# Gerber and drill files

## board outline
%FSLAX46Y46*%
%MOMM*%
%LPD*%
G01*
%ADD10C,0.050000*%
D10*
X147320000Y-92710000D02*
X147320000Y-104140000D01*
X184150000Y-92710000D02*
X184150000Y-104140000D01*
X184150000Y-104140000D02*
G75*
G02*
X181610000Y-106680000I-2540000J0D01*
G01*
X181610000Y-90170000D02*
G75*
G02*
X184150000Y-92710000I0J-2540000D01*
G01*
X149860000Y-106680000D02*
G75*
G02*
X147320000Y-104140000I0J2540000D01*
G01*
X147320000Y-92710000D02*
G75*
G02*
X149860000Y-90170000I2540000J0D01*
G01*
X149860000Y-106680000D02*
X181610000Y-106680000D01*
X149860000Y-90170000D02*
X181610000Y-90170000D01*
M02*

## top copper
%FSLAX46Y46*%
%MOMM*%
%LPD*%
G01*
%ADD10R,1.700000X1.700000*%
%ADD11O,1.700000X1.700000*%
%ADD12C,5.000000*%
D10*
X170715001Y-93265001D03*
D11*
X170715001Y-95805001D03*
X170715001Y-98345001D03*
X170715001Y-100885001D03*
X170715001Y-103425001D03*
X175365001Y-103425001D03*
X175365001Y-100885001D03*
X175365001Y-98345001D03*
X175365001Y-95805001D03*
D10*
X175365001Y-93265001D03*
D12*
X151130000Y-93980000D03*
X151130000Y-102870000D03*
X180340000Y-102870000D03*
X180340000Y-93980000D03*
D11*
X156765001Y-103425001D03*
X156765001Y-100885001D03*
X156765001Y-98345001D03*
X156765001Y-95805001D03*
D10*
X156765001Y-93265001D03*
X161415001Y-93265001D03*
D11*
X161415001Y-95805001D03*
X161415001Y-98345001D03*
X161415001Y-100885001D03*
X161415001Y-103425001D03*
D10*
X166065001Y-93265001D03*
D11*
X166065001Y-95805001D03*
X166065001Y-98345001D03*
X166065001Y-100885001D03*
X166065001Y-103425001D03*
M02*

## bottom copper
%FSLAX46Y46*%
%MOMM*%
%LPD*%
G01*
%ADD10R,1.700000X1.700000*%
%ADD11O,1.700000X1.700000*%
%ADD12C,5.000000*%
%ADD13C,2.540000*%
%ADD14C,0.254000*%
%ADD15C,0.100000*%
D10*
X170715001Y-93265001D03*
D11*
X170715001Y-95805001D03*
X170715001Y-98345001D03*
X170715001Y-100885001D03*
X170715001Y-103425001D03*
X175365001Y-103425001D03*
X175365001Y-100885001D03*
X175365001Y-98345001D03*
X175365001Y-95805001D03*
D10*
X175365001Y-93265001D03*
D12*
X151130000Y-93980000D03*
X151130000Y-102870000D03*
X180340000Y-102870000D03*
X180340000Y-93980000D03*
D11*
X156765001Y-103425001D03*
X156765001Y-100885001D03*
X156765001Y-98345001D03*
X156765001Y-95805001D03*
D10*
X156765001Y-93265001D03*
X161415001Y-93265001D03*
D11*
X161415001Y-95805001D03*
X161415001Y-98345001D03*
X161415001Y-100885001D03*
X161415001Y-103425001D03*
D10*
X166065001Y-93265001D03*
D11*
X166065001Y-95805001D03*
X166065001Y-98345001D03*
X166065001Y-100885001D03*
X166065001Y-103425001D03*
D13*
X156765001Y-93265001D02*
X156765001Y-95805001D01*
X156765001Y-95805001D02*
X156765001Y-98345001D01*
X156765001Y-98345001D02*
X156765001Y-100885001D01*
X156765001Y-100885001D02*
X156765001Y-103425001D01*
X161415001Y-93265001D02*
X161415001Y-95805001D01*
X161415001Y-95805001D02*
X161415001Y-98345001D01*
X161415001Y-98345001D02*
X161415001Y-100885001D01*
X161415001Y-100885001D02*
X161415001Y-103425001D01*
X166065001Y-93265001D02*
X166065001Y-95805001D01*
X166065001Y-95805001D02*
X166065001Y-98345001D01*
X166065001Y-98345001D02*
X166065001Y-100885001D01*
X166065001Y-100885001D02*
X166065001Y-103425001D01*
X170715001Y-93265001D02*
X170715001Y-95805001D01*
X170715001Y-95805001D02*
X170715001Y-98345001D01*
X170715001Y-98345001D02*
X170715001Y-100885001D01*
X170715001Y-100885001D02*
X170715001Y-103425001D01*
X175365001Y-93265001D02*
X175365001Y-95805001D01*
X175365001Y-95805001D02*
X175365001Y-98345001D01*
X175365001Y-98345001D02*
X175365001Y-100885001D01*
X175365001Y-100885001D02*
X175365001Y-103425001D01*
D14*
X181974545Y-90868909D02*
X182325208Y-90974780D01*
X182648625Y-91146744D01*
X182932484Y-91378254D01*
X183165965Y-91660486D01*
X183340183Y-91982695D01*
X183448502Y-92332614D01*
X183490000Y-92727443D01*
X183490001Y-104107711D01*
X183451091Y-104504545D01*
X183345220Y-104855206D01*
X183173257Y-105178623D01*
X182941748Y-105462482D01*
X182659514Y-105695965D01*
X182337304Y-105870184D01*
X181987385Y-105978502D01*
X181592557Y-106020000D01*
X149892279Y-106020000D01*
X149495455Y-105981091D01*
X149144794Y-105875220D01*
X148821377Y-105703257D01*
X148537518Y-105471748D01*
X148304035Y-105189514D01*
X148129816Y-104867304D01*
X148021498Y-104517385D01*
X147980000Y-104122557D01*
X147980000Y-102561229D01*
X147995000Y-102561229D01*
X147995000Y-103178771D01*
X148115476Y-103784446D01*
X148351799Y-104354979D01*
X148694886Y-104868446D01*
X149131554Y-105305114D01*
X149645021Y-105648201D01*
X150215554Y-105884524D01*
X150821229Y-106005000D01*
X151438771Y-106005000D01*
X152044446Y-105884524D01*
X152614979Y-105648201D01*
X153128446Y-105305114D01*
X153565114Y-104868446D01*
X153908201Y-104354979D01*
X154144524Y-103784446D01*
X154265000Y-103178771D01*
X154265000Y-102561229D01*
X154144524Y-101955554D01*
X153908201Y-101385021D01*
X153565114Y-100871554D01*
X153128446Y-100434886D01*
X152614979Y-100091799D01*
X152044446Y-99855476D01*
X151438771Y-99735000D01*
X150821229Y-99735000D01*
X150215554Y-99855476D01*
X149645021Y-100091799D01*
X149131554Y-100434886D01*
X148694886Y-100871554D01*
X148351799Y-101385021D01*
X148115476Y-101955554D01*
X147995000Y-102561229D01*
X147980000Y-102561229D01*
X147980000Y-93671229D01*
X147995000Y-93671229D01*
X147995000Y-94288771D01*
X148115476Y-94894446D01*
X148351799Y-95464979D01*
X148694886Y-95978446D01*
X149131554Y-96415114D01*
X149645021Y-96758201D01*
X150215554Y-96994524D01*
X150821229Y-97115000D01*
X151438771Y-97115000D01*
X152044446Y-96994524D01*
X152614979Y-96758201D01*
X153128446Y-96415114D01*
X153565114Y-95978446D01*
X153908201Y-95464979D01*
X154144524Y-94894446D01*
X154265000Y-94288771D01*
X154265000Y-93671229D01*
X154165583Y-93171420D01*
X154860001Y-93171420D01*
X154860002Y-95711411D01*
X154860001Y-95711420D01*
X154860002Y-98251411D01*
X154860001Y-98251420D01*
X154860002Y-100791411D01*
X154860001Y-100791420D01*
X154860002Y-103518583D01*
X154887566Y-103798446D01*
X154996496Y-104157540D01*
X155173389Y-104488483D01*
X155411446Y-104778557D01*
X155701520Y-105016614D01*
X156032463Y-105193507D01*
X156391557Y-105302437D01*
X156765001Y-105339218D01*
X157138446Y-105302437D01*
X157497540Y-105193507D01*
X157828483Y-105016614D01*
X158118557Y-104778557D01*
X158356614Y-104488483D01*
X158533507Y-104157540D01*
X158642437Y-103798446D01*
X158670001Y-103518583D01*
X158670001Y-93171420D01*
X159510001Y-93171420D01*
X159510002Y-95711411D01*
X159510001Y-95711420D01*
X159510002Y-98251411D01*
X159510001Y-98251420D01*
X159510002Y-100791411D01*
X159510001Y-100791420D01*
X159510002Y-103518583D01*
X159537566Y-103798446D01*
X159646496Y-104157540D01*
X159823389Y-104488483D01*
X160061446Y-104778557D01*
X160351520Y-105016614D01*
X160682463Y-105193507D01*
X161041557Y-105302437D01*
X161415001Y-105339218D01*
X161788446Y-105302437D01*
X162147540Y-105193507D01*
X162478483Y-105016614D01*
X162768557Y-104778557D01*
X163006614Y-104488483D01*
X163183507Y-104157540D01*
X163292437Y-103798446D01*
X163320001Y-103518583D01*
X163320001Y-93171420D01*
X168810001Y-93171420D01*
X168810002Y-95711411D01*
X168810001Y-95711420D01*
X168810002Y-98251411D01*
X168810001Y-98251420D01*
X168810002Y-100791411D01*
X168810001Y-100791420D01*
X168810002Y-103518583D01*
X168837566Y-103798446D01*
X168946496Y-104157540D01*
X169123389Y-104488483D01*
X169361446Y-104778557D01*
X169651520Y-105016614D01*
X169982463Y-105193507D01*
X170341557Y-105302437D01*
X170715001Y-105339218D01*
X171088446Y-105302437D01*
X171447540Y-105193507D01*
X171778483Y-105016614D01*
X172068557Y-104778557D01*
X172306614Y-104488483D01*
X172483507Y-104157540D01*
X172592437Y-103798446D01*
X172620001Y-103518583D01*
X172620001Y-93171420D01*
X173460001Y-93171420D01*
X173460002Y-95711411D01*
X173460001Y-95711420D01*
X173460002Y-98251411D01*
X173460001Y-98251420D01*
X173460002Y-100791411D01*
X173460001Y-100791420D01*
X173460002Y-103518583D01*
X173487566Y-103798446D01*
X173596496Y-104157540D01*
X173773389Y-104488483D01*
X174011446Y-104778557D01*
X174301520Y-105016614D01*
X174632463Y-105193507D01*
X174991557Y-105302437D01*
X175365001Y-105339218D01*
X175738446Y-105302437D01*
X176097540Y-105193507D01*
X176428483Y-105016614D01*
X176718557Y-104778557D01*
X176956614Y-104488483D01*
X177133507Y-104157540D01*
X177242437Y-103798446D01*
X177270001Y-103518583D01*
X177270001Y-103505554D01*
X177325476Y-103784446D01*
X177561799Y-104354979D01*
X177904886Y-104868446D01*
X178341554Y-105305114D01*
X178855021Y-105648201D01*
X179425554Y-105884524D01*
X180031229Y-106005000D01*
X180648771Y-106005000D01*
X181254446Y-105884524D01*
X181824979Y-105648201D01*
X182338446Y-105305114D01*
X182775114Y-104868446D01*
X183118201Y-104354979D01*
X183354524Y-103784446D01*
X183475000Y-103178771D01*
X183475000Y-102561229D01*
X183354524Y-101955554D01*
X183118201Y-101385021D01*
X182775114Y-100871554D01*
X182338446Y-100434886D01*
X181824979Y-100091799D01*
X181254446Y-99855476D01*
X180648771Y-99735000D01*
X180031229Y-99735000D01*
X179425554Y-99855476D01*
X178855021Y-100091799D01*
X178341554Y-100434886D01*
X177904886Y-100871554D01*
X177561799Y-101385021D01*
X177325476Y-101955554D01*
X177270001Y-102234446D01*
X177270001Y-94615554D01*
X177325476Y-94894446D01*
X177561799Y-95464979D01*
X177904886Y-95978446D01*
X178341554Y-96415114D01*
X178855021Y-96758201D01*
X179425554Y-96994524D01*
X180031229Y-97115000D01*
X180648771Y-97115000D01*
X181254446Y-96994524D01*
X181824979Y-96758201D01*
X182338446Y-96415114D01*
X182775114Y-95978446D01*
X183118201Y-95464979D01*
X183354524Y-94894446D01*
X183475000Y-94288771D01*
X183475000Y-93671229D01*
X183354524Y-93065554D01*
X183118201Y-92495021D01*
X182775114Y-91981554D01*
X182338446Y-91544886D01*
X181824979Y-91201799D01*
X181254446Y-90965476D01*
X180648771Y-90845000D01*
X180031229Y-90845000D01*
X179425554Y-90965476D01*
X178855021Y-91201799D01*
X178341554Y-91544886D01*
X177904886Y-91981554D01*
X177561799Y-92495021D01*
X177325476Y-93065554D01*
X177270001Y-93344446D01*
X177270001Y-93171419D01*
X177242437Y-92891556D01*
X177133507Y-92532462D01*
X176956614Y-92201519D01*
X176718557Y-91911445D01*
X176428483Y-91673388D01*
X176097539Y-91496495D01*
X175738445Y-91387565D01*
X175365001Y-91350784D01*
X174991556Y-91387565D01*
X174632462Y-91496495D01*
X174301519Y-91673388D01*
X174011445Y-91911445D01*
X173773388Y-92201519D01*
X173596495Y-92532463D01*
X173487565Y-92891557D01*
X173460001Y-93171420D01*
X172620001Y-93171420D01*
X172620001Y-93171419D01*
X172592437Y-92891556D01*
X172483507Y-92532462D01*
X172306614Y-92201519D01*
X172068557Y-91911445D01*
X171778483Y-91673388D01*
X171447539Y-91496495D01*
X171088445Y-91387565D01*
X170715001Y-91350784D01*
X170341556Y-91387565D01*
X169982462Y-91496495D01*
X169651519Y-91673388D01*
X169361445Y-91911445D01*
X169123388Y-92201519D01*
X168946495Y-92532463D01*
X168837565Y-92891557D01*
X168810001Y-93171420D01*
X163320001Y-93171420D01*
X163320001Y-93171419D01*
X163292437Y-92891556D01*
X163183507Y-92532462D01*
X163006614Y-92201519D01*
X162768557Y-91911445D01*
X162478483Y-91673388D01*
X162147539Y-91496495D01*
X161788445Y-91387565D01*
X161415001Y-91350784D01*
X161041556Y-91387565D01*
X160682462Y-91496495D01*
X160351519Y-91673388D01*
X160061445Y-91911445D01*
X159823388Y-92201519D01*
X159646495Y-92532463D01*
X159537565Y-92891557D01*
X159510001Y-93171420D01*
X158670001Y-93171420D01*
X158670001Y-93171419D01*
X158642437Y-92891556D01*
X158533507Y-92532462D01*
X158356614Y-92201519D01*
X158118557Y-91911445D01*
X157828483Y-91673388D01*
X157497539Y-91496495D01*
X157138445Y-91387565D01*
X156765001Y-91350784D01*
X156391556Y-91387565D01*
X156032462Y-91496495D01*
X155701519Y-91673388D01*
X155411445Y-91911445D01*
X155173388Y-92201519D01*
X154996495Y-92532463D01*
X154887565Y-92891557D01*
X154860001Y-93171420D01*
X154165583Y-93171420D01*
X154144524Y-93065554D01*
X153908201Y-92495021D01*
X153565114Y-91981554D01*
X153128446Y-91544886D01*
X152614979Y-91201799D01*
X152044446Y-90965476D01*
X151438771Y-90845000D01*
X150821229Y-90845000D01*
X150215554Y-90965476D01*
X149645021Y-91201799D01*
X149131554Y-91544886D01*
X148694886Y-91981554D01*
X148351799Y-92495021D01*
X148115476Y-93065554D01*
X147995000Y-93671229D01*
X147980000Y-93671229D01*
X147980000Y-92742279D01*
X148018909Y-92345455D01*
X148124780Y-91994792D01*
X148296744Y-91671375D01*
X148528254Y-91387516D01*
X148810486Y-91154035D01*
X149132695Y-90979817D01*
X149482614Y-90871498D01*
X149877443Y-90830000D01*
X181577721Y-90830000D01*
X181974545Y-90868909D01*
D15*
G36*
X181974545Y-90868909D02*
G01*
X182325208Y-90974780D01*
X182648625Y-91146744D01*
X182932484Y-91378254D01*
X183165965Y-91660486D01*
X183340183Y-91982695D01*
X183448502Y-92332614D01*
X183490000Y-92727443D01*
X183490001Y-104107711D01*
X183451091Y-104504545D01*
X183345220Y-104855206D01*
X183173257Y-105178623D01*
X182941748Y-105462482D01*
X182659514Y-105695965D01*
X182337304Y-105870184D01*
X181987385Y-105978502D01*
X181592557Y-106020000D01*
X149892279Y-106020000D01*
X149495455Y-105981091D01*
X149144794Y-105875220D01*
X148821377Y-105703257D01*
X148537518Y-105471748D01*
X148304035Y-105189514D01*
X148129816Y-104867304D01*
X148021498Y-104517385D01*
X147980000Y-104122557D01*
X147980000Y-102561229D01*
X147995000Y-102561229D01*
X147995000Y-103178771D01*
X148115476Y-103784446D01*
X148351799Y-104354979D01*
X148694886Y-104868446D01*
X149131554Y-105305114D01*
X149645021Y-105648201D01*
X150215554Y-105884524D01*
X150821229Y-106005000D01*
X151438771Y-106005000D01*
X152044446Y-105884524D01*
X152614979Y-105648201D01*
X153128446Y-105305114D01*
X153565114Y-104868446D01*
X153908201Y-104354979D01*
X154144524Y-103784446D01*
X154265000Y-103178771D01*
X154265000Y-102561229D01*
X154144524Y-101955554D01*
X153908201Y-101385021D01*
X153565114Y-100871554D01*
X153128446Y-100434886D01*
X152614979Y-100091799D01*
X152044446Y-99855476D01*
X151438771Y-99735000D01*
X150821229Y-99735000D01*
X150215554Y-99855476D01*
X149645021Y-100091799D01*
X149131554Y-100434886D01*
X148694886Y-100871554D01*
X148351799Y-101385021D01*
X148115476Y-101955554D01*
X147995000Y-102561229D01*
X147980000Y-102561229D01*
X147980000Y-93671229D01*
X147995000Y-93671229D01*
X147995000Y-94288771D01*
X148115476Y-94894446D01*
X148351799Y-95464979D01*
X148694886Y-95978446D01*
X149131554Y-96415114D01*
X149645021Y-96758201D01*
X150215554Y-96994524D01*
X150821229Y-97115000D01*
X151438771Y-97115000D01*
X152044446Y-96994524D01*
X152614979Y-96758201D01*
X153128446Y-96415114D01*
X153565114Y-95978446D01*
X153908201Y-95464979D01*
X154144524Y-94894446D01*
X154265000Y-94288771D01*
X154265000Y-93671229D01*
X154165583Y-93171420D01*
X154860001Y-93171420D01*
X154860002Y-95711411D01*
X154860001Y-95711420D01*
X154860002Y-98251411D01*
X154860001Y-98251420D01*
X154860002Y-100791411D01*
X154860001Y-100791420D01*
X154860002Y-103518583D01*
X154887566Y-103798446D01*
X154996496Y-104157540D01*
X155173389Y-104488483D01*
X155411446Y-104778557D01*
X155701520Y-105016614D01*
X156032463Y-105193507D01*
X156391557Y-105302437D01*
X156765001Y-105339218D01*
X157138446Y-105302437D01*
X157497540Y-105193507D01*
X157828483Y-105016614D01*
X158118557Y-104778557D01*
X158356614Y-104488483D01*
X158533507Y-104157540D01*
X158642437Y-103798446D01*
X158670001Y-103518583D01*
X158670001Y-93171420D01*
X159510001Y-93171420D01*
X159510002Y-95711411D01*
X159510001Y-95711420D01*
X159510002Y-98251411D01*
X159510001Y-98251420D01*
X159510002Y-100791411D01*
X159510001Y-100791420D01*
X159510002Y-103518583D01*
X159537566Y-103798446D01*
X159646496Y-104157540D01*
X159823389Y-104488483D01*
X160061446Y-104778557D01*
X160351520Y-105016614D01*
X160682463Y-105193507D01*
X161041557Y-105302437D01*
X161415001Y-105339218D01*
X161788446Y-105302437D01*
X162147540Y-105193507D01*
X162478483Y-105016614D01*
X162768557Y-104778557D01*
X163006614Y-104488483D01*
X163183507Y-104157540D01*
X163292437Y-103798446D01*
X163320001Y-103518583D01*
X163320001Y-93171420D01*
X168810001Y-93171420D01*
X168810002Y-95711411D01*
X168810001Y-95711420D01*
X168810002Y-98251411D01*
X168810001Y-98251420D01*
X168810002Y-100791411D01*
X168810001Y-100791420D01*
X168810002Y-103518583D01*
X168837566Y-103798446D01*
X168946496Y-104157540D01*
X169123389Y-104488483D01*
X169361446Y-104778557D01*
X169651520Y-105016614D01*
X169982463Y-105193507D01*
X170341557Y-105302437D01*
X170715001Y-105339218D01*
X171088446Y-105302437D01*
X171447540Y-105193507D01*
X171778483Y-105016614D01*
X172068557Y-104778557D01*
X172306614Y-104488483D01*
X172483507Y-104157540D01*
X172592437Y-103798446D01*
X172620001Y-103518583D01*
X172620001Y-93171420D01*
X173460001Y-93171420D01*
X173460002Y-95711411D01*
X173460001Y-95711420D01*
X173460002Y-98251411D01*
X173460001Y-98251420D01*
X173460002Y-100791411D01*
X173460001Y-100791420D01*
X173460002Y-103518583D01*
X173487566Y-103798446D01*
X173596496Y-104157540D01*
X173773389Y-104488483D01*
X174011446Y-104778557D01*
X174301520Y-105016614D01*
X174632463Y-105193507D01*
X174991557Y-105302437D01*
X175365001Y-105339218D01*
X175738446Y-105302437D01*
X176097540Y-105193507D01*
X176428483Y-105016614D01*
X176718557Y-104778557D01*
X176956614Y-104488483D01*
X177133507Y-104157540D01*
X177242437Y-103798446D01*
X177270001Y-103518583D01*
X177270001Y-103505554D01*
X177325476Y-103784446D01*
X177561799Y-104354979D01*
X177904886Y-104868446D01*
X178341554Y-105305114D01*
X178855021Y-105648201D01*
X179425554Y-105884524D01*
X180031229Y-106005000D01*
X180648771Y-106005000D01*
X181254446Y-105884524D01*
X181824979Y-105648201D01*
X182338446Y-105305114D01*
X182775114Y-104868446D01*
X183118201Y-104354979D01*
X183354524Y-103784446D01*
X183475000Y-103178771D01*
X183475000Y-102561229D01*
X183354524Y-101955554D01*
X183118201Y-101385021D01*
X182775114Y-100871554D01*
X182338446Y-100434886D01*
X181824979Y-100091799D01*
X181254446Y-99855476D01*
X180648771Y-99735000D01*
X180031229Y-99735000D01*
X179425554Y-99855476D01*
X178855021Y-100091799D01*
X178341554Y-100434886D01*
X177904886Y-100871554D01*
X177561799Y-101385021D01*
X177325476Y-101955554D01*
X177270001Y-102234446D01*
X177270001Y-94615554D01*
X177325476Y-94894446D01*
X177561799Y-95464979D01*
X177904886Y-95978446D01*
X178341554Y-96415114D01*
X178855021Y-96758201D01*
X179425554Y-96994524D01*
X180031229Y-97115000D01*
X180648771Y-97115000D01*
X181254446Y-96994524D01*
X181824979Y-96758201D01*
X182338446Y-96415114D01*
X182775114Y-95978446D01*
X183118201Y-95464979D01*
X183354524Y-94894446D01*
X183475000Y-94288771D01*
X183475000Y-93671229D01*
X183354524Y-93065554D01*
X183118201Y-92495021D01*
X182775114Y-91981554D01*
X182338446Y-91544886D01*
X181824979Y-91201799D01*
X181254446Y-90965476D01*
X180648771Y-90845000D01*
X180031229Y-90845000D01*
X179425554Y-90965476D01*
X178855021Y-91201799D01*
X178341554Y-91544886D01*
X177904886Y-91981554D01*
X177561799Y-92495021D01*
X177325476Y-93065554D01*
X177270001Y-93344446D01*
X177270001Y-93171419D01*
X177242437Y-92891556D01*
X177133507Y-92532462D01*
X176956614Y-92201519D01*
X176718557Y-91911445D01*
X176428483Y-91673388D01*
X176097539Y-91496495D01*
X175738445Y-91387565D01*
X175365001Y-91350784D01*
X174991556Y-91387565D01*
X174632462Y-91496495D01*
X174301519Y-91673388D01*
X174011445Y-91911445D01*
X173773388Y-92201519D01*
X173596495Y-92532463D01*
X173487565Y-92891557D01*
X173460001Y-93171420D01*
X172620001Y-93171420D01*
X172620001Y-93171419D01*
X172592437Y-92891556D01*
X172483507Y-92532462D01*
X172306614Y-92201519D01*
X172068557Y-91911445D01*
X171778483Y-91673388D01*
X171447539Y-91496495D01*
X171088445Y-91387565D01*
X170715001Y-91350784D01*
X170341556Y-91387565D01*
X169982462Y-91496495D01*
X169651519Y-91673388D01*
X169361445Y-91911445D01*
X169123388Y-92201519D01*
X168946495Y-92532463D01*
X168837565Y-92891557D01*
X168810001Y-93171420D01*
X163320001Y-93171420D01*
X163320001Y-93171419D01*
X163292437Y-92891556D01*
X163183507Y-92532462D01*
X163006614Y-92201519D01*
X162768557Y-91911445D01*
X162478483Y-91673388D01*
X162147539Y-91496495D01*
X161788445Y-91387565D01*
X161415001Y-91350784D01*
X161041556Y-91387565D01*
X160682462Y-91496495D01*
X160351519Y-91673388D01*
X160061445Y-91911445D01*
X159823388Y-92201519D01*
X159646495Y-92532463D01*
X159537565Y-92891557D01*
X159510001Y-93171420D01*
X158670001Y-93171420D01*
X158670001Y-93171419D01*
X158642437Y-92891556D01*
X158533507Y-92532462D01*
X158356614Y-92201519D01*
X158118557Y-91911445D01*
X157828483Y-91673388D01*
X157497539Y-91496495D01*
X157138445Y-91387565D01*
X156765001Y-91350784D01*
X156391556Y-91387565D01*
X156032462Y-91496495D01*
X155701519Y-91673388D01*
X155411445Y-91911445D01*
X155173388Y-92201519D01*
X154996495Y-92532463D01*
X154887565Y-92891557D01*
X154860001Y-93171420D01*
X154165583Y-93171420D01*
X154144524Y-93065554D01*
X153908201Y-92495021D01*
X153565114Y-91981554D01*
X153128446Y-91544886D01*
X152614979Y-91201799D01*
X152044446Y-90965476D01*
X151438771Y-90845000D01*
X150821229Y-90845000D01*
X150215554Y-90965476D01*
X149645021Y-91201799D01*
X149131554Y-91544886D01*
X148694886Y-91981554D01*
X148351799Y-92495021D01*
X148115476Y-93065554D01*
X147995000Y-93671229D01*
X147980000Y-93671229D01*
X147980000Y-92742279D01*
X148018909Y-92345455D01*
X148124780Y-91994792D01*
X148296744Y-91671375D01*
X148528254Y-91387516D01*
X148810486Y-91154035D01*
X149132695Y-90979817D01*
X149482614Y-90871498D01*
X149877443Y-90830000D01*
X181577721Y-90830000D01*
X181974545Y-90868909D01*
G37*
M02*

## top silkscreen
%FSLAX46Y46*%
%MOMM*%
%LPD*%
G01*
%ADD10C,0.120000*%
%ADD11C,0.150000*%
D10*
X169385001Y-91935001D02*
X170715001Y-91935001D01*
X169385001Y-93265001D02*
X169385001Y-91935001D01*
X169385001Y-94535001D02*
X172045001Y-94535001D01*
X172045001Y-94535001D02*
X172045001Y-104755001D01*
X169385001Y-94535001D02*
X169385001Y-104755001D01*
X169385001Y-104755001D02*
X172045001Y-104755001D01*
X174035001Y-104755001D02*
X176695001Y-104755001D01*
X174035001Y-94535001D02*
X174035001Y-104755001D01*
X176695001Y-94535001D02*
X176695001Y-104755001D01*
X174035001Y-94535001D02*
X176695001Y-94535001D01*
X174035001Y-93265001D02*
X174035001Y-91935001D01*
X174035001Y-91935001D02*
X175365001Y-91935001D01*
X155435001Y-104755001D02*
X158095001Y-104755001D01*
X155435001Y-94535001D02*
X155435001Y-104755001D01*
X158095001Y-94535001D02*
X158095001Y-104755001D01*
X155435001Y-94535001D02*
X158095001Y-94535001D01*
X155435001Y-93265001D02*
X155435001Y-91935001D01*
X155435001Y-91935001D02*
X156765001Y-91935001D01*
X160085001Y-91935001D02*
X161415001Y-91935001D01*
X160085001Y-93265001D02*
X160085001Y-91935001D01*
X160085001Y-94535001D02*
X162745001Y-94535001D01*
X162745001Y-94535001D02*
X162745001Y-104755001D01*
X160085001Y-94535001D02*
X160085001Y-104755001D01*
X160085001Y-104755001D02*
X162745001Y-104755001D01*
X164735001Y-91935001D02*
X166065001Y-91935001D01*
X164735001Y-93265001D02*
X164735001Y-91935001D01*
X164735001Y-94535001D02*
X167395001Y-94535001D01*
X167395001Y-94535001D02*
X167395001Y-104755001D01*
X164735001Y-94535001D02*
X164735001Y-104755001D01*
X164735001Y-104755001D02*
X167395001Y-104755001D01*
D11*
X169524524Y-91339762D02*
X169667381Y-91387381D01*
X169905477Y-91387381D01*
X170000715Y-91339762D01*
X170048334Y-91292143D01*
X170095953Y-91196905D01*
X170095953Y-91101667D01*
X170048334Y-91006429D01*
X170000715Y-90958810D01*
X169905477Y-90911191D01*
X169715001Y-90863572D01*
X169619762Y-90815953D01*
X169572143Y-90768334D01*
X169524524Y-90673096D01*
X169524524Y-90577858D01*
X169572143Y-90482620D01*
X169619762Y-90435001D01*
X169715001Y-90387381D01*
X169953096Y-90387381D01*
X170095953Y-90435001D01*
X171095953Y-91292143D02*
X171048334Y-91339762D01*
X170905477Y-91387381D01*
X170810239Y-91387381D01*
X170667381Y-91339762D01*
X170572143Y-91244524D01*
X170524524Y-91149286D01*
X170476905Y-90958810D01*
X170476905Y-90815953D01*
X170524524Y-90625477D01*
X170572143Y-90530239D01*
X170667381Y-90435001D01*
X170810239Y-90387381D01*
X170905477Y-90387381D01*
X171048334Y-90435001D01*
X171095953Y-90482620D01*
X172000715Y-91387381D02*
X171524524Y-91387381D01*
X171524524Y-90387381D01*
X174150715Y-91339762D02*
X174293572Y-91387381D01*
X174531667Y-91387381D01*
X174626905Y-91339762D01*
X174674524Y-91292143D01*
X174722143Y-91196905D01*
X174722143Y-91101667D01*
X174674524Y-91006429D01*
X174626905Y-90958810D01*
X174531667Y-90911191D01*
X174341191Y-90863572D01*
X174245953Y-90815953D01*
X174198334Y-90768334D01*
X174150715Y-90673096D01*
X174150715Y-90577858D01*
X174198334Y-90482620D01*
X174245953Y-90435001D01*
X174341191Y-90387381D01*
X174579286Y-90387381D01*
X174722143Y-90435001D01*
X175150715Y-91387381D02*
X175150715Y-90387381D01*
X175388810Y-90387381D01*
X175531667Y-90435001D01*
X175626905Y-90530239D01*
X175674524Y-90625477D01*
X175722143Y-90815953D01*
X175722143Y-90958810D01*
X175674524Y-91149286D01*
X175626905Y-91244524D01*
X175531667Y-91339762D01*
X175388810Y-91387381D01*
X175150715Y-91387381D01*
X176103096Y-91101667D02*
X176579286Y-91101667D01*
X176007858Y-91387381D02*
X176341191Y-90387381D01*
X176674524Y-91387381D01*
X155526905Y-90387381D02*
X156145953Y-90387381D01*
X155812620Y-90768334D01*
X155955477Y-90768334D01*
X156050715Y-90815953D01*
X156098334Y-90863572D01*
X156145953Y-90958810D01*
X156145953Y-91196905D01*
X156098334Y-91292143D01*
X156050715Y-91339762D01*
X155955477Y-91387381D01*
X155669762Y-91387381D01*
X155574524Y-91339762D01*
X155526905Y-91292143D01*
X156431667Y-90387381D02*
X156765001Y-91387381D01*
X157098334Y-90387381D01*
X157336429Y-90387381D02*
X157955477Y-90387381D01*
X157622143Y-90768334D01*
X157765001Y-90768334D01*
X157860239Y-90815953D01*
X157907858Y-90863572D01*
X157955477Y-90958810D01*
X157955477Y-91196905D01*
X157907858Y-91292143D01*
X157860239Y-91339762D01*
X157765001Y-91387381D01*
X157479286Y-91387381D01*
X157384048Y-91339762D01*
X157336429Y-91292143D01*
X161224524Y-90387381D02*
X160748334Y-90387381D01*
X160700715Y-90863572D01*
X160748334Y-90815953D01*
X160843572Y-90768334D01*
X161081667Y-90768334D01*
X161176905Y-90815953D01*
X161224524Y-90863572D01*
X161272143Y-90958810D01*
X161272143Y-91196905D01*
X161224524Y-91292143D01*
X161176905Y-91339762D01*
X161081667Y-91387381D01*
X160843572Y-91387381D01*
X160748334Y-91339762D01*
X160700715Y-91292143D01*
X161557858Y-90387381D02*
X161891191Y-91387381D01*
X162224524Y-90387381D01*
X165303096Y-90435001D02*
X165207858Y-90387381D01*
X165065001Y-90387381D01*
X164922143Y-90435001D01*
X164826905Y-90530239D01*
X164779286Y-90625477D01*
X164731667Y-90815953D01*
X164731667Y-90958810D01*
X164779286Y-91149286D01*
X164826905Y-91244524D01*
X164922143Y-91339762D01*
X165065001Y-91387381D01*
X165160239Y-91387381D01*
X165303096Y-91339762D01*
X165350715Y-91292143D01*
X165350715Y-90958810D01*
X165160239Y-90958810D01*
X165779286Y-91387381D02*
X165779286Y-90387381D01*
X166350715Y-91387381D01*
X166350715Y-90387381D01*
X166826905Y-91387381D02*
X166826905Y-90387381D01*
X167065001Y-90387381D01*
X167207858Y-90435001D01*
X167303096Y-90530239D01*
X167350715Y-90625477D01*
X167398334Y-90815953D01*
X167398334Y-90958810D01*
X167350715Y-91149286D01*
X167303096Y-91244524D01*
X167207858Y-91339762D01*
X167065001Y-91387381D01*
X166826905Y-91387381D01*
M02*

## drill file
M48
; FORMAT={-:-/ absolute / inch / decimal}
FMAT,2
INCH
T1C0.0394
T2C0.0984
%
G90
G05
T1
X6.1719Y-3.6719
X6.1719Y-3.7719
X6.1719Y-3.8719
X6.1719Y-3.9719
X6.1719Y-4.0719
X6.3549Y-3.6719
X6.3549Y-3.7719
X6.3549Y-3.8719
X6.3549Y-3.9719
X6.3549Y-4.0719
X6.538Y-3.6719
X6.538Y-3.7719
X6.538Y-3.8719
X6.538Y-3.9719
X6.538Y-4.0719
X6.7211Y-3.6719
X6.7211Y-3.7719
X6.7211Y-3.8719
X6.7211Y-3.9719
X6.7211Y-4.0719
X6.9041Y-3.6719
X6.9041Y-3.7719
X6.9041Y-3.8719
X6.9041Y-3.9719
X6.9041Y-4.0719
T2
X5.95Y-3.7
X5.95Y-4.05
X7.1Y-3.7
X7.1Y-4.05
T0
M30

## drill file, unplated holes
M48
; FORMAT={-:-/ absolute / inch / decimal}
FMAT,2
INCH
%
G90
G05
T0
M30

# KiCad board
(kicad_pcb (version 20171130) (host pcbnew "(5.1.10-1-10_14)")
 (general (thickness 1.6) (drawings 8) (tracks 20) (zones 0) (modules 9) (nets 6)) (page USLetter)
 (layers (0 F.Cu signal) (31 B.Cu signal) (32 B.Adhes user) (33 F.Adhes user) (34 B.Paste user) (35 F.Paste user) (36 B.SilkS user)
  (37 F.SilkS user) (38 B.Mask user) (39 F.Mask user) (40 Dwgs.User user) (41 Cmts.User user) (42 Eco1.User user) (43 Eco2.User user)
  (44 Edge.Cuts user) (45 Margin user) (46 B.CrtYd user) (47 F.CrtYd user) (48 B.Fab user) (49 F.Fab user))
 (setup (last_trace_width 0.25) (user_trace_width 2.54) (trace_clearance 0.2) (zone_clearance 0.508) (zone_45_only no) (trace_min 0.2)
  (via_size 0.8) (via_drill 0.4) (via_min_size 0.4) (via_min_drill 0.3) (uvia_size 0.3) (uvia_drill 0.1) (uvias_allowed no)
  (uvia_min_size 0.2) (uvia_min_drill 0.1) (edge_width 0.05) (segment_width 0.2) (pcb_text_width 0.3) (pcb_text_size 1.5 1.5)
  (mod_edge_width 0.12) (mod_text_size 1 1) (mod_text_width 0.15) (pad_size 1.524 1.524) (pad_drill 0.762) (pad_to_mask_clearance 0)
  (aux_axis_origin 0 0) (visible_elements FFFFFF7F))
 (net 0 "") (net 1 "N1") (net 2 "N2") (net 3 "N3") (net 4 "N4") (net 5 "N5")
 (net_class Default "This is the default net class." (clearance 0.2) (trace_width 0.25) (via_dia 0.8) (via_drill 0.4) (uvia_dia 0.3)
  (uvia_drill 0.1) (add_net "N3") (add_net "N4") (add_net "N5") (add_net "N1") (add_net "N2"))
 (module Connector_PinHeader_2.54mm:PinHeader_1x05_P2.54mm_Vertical (layer F.Cu) (at 170.715001 93.265001)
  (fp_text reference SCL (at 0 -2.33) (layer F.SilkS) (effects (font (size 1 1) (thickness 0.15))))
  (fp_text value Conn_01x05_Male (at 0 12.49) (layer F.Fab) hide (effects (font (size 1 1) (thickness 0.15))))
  (fp_line (start -1.33 11.49) (end 1.33 11.49) (layer F.SilkS) (width 0.12))
  (fp_line (start -1.33 1.27) (end -1.33 11.49) (layer F.SilkS) (width 0.12))
  (fp_line (start 1.33 1.27) (end 1.33 11.49) (layer F.SilkS) (width 0.12))
  (fp_line (start -1.33 1.27) (end 1.33 1.27) (layer F.SilkS) (width 0.12))
  (fp_line (start -1.33 0) (end -1.33 -1.33) (layer F.SilkS) (width 0.12))
  (fp_line (start -1.33 -1.33) (end 0 -1.33) (layer F.SilkS) (width 0.12))
  (pad 1 thru_hole rect (at 0 0) (size 1.7 1.7) (drill 1) (layers *.Cu *.Mask) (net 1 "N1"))
  (pad 2 thru_hole oval (at 0 2.54) (size 1.7 1.7) (drill 1) (layers *.Cu *.Mask) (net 1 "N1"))
  (pad 3 thru_hole oval (at 0 5.08) (size 1.7 1.7) (drill 1) (layers *.Cu *.Mask) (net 1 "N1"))
  (pad 4 thru_hole oval (at 0 7.62) (size 1.7 1.7) (drill 1) (layers *.Cu *.Mask) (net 1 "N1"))
  (pad 5 thru_hole oval (at 0 10.16) (size 1.7 1.7) (drill 1) (layers *.Cu *.Mask) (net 1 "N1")))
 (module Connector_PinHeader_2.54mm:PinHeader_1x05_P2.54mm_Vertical (layer F.Cu) (at 175.365001 93.265001)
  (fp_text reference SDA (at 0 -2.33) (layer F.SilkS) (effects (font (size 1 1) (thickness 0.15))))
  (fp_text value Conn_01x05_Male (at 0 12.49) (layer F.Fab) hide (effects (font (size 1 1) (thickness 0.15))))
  (fp_line (start -1.33 -1.33) (end 0 -1.33) (layer F.SilkS) (width 0.12))
  (fp_line (start -1.33 0) (end -1.33 -1.33) (layer F.SilkS) (width 0.12))
  (fp_line (start -1.33 1.27) (end 1.33 1.27) (layer F.SilkS) (width 0.12))
  (fp_line (start 1.33 1.27) (end 1.33 11.49) (layer F.SilkS) (width 0.12))
  (fp_line (start -1.33 1.27) (end -1.33 11.49) (layer F.SilkS) (width 0.12))
  (fp_line (start -1.33 11.49) (end 1.33 11.49) (layer F.SilkS) (width 0.12))
  (pad 5 thru_hole oval (at 0 10.16) (size 1.7 1.7) (drill 1) (layers *.Cu *.Mask) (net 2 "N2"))
  (pad 4 thru_hole oval (at 0 7.62) (size 1.7 1.7) (drill 1) (layers *.Cu *.Mask) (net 2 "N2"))
  (pad 3 thru_hole oval (at 0 5.08) (size 1.7 1.7) (drill 1) (layers *.Cu *.Mask) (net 2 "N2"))
  (pad 2 thru_hole oval (at 0 2.54) (size 1.7 1.7) (drill 1) (layers *.Cu *.Mask) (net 2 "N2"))
  (pad 1 thru_hole rect (at 0 0) (size 1.7 1.7) (drill 1) (layers *.Cu *.Mask) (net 2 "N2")))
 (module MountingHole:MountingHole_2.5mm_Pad (layer F.Cu) (at 151.13 93.98)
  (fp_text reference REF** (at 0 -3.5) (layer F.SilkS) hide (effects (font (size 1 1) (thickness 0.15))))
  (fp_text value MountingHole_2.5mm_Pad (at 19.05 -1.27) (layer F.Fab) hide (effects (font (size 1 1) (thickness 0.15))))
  (pad 1 thru_hole circle (at 0 0) (size 5 5) (drill 2.5) (layers *.Cu *.Mask)))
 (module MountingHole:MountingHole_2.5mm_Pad (layer F.Cu) (at 151.13 102.87)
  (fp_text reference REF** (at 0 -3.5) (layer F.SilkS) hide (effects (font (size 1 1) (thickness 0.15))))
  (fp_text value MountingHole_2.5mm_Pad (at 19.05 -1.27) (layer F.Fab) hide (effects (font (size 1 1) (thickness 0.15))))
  (pad 1 thru_hole circle (at 0 0) (size 5 5) (drill 2.5) (layers *.Cu *.Mask)))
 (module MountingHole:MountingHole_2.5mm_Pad (layer F.Cu) (at 180.34 102.87)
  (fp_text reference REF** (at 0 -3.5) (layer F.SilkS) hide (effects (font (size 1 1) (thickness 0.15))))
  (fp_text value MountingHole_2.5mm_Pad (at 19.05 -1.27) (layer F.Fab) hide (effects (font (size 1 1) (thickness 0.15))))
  (pad 1 thru_hole circle (at 0 0) (size 5 5) (drill 2.5) (layers *.Cu *.Mask)))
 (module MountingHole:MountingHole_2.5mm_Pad (layer F.Cu) (at 180.34 93.98)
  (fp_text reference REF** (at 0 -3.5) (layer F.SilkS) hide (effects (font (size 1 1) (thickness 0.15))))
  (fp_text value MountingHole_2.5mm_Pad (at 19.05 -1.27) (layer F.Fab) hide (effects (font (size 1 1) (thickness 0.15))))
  (pad 1 thru_hole circle (at 0 0) (size 5 5) (drill 2.5) (layers *.Cu *.Mask)))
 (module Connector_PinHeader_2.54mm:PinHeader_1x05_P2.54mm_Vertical (layer F.Cu) (at 156.765001 93.265001)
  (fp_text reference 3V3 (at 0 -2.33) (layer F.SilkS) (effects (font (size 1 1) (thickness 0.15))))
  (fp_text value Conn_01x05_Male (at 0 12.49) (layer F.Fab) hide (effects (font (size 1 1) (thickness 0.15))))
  (fp_line (start -1.33 -1.33) (end 0 -1.33) (layer F.SilkS) (width 0.12))
  (fp_line (start -1.33 0) (end -1.33 -1.33) (layer F.SilkS) (width 0.12))
  (fp_line (start -1.33 1.27) (end 1.33 1.27) (layer F.SilkS) (width 0.12))
  (fp_line (start 1.33 1.27) (end 1.33 11.49) (layer F.SilkS) (width 0.12))
  (fp_line (start -1.33 1.27) (end -1.33 11.49) (layer F.SilkS) (width 0.12))
  (fp_line (start -1.33 11.49) (end 1.33 11.49) (layer F.SilkS) (width 0.12))
  (pad 5 thru_hole oval (at 0 10.16) (size 1.7 1.7) (drill 1) (layers *.Cu *.Mask) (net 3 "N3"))
  (pad 4 thru_hole oval (at 0 7.62) (size 1.7 1.7) (drill 1) (layers *.Cu *.Mask) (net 3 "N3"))
  (pad 3 thru_hole oval (at 0 5.08) (size 1.7 1.7) (drill 1) (layers *.Cu *.Mask) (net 3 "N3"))
  (pad 2 thru_hole oval (at 0 2.54) (size 1.7 1.7) (drill 1) (layers *.Cu *.Mask) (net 3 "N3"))
  (pad 1 thru_hole rect (at 0 0) (size 1.7 1.7) (drill 1) (layers *.Cu *.Mask) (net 3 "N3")))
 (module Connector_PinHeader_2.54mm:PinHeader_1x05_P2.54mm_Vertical (layer F.Cu) (at 161.415001 93.265001)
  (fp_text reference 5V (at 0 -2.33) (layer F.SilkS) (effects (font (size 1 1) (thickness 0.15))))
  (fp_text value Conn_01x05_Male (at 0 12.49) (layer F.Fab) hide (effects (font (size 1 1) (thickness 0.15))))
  (fp_line (start -1.33 11.49) (end 1.33 11.49) (layer F.SilkS) (width 0.12))
  (fp_line (start -1.33 1.27) (end -1.33 11.49) (layer F.SilkS) (width 0.12))
  (fp_line (start 1.33 1.27) (end 1.33 11.49) (layer F.SilkS) (width 0.12))
  (fp_line (start -1.33 1.27) (end 1.33 1.27) (layer F.SilkS) (width 0.12))
  (fp_line (start -1.33 0) (end -1.33 -1.33) (layer F.SilkS) (width 0.12))
  (fp_line (start -1.33 -1.33) (end 0 -1.33) (layer F.SilkS) (width 0.12))
  (pad 1 thru_hole rect (at 0 0) (size 1.7 1.7) (drill 1) (layers *.Cu *.Mask) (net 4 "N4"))
  (pad 2 thru_hole oval (at 0 2.54) (size 1.7 1.7) (drill 1) (layers *.Cu *.Mask) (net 4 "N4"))
  (pad 3 thru_hole oval (at 0 5.08) (size 1.7 1.7) (drill 1) (layers *.Cu *.Mask) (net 4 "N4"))
  (pad 4 thru_hole oval (at 0 7.62) (size 1.7 1.7) (drill 1) (layers *.Cu *.Mask) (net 4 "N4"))
  (pad 5 thru_hole oval (at 0 10.16) (size 1.7 1.7) (drill 1) (layers *.Cu *.Mask) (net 4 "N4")))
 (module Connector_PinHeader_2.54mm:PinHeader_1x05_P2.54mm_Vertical (layer F.Cu) (at 166.065001 93.265001)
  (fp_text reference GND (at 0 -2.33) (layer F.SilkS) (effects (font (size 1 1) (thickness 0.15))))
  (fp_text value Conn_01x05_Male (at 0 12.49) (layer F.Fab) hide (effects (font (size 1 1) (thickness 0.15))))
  (fp_line (start -1.33 11.49) (end 1.33 11.49) (layer F.SilkS) (width 0.12))
  (fp_line (start -1.33 1.27) (end -1.33 11.49) (layer F.SilkS) (width 0.12))
  (fp_line (start 1.33 1.27) (end 1.33 11.49) (layer F.SilkS) (width 0.12))
  (fp_line (start -1.33 1.27) (end 1.33 1.27) (layer F.SilkS) (width 0.12))
  (fp_line (start -1.33 0) (end -1.33 -1.33) (layer F.SilkS) (width 0.12))
  (fp_line (start -1.33 -1.33) (end 0 -1.33) (layer F.SilkS) (width 0.12))
  (pad 1 thru_hole rect (at 0 0) (size 1.7 1.7) (drill 1) (layers *.Cu *.Mask) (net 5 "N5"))
  (pad 2 thru_hole oval (at 0 2.54) (size 1.7 1.7) (drill 1) (layers *.Cu *.Mask) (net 5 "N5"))
  (pad 3 thru_hole oval (at 0 5.08) (size 1.7 1.7) (drill 1) (layers *.Cu *.Mask) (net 5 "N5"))
  (pad 4 thru_hole oval (at 0 7.62) (size 1.7 1.7) (drill 1) (layers *.Cu *.Mask) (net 5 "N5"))
  (pad 5 thru_hole oval (at 0 10.16) (size 1.7 1.7) (drill 1) (layers *.Cu *.Mask) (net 5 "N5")))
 (gr_line (start 147.32 92.71) (end 147.32 104.14) (layer Edge.Cuts) (width 0.05))
 (gr_line (start 184.15 92.71) (end 184.15 104.14) (layer Edge.Cuts) (width 0.05))
 (gr_arc (start 181.61 104.14) (end 181.61 106.68) (angle -90) (layer Edge.Cuts) (width 0.05))
 (gr_arc (start 181.61 92.71) (end 184.15 92.71) (angle -90) (layer Edge.Cuts) (width 0.05))
 (gr_arc (start 149.86 104.14) (end 147.32 104.14) (angle -90) (layer Edge.Cuts) (width 0.05))
 (gr_arc (start 149.86 92.71) (end 149.86 90.17) (angle -90) (layer Edge.Cuts) (width 0.05))
 (gr_line (start 149.86 106.68) (end 181.61 106.68) (layer Edge.Cuts) (width 0.05))
 (gr_line (start 149.86 90.17) (end 181.61 90.17) (layer Edge.Cuts) (width 0.05))
 (segment (start 156.765001 93.265001) (end 156.765001 95.805001) (width 2.54) (layer B.Cu) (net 3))
 (segment (start 156.765001 95.805001) (end 156.765001 98.345001) (width 2.54) (layer B.Cu) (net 3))
 (segment (start 156.765001 98.345001) (end 156.765001 100.885001) (width 2.54) (layer B.Cu) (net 3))
 (segment (start 156.765001 100.885001) (end 156.765001 103.425001) (width 2.54) (layer B.Cu) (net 3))
 (segment (start 161.415001 93.265001) (end 161.415001 95.805001) (width 2.54) (layer B.Cu) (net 4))
 (segment (start 161.415001 95.805001) (end 161.415001 98.345001) (width 2.54) (layer B.Cu) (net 4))
 (segment (start 161.415001 98.345001) (end 161.415001 100.885001) (width 2.54) (layer B.Cu) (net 4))
 (segment (start 161.415001 100.885001) (end 161.415001 103.425001) (width 2.54) (layer B.Cu) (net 4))
 (segment (start 166.065001 93.265001) (end 166.065001 95.805001) (width 2.54) (layer B.Cu) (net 5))
 (segment (start 166.065001 95.805001) (end 166.065001 98.345001) (width 2.54) (layer B.Cu) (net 5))
 (segment (start 166.065001 98.345001) (end 166.065001 100.885001) (width 2.54) (layer B.Cu) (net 5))
 (segment (start 166.065001 100.885001) (end 166.065001 103.425001) (width 2.54) (layer B.Cu) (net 5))
 (segment (start 170.715001 93.265001) (end 170.715001 95.805001) (width 2.54) (layer B.Cu) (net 1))
 (segment (start 170.715001 95.805001) (end 170.715001 98.345001) (width 2.54) (layer B.Cu) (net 1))
 (segment (start 170.715001 98.345001) (end 170.715001 100.885001) (width 2.54) (layer B.Cu) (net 1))
 (segment (start 170.715001 100.885001) (end 170.715001 103.425001) (width 2.54) (layer B.Cu) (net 1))
 (segment (start 175.365001 93.265001) (end 175.365001 95.805001) (width 2.54) (layer B.Cu) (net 2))
 (segment (start 175.365001 95.805001) (end 175.365001 98.345001) (width 2.54) (layer B.Cu) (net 2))
 (segment (start 175.365001 98.345001) (end 175.365001 100.885001) (width 2.54) (layer B.Cu) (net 2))
 (segment (start 175.365001 100.885001) (end 175.365001 103.425001) (width 2.54) (layer B.Cu) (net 2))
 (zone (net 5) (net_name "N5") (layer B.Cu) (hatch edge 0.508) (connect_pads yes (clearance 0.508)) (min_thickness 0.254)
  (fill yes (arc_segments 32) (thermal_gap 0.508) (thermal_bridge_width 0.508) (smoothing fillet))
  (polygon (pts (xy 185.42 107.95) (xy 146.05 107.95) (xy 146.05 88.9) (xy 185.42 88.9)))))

